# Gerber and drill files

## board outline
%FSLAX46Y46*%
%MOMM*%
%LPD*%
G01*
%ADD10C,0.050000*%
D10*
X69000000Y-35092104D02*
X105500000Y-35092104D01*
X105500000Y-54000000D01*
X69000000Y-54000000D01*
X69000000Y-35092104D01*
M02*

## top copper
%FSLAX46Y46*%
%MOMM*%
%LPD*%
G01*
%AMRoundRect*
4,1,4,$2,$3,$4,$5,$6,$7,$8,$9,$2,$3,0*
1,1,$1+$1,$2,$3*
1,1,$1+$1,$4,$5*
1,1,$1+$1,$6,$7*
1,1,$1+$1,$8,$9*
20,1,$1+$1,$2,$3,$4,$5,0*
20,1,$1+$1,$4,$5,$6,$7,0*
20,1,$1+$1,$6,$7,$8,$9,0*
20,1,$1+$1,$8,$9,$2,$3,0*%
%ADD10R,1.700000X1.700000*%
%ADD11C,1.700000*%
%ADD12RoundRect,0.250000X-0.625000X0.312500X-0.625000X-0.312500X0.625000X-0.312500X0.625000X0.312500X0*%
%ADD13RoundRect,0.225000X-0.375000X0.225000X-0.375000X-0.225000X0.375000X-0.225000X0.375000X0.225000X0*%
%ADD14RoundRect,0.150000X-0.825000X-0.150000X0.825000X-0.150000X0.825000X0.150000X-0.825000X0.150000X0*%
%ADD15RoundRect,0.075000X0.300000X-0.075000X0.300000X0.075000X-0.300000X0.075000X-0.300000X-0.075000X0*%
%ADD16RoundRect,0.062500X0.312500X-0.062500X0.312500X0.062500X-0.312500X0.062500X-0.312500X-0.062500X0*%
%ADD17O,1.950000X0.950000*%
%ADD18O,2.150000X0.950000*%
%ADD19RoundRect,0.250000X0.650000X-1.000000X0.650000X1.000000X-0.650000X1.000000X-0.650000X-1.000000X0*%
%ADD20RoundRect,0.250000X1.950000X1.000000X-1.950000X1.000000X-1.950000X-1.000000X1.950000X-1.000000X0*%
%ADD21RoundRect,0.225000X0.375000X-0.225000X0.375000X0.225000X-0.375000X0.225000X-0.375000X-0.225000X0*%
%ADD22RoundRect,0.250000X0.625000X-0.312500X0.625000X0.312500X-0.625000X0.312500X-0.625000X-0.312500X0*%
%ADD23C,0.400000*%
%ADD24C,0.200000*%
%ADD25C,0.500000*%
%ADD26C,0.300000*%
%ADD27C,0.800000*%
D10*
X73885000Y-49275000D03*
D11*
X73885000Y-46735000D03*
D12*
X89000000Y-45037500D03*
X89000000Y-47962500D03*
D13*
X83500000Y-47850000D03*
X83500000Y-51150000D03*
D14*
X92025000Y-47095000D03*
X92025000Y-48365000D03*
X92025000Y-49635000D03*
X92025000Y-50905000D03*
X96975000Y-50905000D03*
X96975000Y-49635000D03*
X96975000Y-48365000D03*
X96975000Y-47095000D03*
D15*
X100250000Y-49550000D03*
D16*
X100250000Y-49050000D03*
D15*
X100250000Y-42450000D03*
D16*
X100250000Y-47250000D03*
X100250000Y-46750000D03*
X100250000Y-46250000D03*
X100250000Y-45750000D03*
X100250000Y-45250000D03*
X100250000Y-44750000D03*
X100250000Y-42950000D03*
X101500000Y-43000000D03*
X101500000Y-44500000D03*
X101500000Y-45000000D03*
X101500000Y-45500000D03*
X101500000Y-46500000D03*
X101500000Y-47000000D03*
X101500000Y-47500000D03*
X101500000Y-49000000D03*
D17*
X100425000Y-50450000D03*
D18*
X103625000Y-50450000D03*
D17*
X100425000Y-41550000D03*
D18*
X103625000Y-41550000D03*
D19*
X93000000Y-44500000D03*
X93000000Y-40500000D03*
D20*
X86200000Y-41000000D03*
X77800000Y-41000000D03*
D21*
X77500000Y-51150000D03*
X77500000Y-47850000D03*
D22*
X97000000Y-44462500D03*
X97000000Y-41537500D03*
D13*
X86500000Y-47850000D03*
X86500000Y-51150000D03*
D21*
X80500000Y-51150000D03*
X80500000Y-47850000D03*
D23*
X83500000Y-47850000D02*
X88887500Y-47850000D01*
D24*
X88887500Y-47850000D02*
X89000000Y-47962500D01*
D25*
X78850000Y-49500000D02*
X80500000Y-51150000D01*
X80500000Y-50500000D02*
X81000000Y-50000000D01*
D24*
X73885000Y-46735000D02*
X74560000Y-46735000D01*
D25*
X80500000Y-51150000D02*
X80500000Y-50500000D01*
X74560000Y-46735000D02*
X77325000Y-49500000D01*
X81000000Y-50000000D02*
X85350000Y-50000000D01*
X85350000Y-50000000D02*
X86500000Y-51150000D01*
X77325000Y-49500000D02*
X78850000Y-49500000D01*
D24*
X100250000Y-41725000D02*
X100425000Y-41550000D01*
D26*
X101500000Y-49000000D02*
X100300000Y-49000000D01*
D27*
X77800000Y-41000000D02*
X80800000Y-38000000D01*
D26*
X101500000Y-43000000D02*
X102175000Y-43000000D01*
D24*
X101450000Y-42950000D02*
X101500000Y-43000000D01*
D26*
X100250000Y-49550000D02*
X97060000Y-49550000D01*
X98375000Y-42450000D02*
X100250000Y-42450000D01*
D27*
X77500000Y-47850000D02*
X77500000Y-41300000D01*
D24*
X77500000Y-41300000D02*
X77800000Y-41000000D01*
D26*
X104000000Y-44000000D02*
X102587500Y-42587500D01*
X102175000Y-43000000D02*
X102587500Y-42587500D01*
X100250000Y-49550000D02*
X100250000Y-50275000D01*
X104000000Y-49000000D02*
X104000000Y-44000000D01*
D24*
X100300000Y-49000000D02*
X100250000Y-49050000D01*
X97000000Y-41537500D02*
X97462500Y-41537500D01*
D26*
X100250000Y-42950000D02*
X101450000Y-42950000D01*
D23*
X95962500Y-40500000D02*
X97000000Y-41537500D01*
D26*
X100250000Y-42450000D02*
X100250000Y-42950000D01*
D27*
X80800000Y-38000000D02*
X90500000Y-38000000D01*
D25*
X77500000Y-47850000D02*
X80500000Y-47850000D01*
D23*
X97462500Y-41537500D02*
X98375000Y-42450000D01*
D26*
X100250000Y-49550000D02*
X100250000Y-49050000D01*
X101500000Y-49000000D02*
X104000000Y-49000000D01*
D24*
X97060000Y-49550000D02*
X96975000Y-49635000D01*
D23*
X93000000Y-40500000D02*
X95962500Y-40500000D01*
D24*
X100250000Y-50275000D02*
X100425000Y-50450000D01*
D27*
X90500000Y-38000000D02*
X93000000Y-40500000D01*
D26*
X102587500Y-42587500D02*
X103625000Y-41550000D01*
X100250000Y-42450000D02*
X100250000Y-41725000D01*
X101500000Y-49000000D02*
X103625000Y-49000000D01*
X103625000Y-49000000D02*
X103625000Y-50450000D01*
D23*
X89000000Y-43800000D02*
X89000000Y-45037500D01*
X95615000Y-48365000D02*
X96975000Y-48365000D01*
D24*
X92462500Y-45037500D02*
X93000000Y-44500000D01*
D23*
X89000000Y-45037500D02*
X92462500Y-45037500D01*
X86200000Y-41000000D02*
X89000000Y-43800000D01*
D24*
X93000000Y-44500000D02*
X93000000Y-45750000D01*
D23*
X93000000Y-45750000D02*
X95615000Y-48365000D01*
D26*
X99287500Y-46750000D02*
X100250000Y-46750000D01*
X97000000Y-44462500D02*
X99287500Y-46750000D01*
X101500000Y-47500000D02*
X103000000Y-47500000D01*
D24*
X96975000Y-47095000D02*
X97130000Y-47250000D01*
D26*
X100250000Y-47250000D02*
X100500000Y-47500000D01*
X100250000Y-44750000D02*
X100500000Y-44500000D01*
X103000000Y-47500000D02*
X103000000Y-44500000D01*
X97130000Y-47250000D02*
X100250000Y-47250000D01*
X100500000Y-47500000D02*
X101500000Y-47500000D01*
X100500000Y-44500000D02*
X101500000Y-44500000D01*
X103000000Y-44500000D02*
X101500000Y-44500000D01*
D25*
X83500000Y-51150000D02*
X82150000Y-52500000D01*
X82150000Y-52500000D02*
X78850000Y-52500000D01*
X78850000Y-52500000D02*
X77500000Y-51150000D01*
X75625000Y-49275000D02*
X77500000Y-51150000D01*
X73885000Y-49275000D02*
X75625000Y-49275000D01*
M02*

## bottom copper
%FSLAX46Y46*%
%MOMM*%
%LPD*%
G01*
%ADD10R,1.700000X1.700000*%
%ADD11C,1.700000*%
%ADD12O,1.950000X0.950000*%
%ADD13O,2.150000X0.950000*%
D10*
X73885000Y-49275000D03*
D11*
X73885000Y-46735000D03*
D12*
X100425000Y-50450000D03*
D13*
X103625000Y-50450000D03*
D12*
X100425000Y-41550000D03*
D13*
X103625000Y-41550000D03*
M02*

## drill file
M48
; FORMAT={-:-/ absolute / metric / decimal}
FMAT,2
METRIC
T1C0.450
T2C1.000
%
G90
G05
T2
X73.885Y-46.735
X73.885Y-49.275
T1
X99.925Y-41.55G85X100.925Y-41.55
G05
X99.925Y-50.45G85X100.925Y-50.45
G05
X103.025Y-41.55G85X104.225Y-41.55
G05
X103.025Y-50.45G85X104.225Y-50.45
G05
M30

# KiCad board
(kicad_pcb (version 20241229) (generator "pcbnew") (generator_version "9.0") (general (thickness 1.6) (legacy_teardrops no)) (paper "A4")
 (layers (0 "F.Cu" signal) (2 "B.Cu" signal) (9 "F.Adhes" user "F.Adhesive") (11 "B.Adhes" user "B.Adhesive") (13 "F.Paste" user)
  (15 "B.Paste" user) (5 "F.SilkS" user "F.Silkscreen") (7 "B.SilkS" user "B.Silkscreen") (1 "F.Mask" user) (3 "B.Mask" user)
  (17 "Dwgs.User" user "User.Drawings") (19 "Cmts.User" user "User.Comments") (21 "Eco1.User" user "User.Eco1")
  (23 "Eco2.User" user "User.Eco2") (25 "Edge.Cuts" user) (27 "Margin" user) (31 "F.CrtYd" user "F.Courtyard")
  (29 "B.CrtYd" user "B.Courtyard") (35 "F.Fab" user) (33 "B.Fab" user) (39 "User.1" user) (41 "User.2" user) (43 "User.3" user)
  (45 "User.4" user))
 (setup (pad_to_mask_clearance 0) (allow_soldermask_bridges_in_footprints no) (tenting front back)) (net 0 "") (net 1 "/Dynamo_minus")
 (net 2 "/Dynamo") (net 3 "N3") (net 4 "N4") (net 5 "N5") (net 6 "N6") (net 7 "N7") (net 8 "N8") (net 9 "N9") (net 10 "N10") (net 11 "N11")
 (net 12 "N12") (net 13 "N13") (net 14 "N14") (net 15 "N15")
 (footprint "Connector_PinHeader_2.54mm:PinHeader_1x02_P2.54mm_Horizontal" (layer "F.Cu") (at 73.885 49.275 180)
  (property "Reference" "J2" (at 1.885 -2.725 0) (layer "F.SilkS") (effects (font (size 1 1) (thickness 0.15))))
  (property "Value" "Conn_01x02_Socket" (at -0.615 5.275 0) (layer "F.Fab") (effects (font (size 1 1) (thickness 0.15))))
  (pad "1" thru_hole rect (at 0 0 180) (size 1.7 1.7) (drill 1) (layers "*.Cu" "*.Mask") (remove_unused_layers no) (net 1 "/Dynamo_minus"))
  (pad "2" thru_hole circle (at 0 2.54 180) (size 1.7 1.7) (drill 1) (layers "*.Cu" "*.Mask") (remove_unused_layers no) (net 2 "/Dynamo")))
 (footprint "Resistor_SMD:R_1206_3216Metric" (layer "F.Cu") (at 89 46.5 -90)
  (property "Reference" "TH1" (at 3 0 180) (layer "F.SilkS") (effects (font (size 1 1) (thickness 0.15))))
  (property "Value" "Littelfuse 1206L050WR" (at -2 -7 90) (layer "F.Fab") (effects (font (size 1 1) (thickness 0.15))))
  (pad "1" smd roundrect (at -1.4625 0 270) (size 1.125 1.75) (layers "F.Cu" "F.Mask" "F.Paste") (roundrect_rratio 0.222222) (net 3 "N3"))
  (pad "2" smd roundrect (at 1.4625 0 270) (size 1.125 1.75) (layers "F.Cu" "F.Mask" "F.Paste") (roundrect_rratio 0.222222) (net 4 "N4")))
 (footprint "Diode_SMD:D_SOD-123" (layer "F.Cu") (at 83.5 49.5 -90)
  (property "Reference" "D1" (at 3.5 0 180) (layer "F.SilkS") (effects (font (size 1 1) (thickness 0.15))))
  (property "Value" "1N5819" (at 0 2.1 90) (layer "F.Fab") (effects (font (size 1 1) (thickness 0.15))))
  (pad "1" smd roundrect (at -1.65 0 270) (size 0.9 1.2) (layers "F.Cu" "F.Mask" "F.Paste") (roundrect_rratio 0.25) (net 4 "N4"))
  (pad "2" smd roundrect (at 1.65 0 270) (size 0.9 1.2) (layers "F.Cu" "F.Mask" "F.Paste") (roundrect_rratio 0.25) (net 1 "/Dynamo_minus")))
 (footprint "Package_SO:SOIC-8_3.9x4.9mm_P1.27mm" (layer "F.Cu") (at 94.5 49)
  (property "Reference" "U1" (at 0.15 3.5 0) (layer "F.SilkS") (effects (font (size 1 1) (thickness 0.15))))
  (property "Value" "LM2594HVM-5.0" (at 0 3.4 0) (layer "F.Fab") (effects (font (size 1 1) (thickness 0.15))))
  (pad "1" smd roundrect (at -2.475 -1.905) (size 1.95 0.6) (layers "F.Cu" "F.Mask" "F.Paste") (roundrect_rratio 0.25) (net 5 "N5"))
  (pad "2" smd roundrect (at -2.475 -0.635) (size 1.95 0.6) (layers "F.Cu" "F.Mask" "F.Paste") (roundrect_rratio 0.25) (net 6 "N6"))
  (pad "3" smd roundrect (at -2.475 0.635) (size 1.95 0.6) (layers "F.Cu" "F.Mask" "F.Paste") (roundrect_rratio 0.25) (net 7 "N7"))
  (pad "4" smd roundrect (at -2.475 1.905) (size 1.95 0.6) (layers "F.Cu" "F.Mask" "F.Paste") (roundrect_rratio 0.25) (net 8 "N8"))
  (pad "5" smd roundrect (at 2.475 1.905) (size 1.95 0.6) (layers "F.Cu" "F.Mask" "F.Paste") (roundrect_rratio 0.25) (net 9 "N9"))
  (pad "6" smd roundrect (at 2.475 0.635) (size 1.95 0.6) (layers "F.Cu" "F.Mask" "F.Paste") (roundrect_rratio 0.25) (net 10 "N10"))
  (pad "7" smd roundrect (at 2.475 -0.635) (size 1.95 0.6) (layers "F.Cu" "F.Mask" "F.Paste") (roundrect_rratio 0.25) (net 3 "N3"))
  (pad "8" smd roundrect (at 2.475 -1.905) (size 1.95 0.6) (layers "F.Cu" "F.Mask" "F.Paste") (roundrect_rratio 0.25) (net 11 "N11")))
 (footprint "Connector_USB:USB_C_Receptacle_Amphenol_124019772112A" (layer "F.Cu") (at 103.45 46 90)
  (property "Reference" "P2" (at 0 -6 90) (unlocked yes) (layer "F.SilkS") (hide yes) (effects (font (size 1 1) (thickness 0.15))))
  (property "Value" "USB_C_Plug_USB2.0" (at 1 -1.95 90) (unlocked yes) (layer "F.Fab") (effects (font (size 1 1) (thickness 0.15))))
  (pad "A1" smd roundrect (at -3.55 -3.2 90) (size 0.3 0.75) (layers "F.Cu" "F.Mask" "F.Paste") (roundrect_rratio 0.25) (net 10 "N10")
   (thermal_bridge_angle 45))
  (pad "A1" smd roundrect (at -3.05 -3.2 90) (size 0.25 0.75) (layers "F.Cu" "F.Mask" "F.Paste") (roundrect_rratio 0.25) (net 10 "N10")
   (thermal_bridge_angle 45))
  (pad "A1" smd roundrect (at 3.55 -3.2 90) (size 0.3 0.75) (layers "F.Cu" "F.Mask" "F.Paste") (roundrect_rratio 0.25) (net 10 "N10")
   (thermal_bridge_angle 45))
  (pad "A4" smd roundrect (at -1.25 -3.2 90) (size 0.25 0.75) (layers "F.Cu" "F.Mask" "F.Paste") (roundrect_rratio 0.25) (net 11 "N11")
   (thermal_bridge_angle 45))
  (pad "A5" smd roundrect (at -0.75 -3.2 90) (size 0.25 0.75) (layers "F.Cu" "F.Mask" "F.Paste") (roundrect_rratio 0.25) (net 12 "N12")
   (thermal_bridge_angle 45))
  (pad "A6" smd roundrect (at -0.25 -3.2 90) (size 0.25 0.75) (layers "F.Cu" "F.Mask" "F.Paste") (roundrect_rratio 0.25) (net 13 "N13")
   (thermal_bridge_angle 45))
  (pad "A7" smd roundrect (at 0.25 -3.2 90) (size 0.25 0.75) (layers "F.Cu" "F.Mask" "F.Paste") (roundrect_rratio 0.25) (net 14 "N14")
   (thermal_bridge_angle 45))
  (pad "A8" smd roundrect (at 0.75 -3.2 90) (size 0.25 0.75) (layers "F.Cu" "F.Mask" "F.Paste") (roundrect_rratio 0.25)
   (thermal_bridge_angle 45))
  (pad "A9" smd roundrect (at 1.25 -3.2 90) (size 0.25 0.75) (layers "F.Cu" "F.Mask" "F.Paste") (roundrect_rratio 0.25) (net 11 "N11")
   (thermal_bridge_angle 45))
  (pad "A12" smd roundrect (at 3.05 -3.2 90) (size 0.25 0.75) (layers "F.Cu" "F.Mask" "F.Paste") (roundrect_rratio 0.25) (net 10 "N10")
   (thermal_bridge_angle 45))
  (pad "B1" smd roundrect (at 3 -1.95 90) (size 0.25 0.75) (layers "F.Cu" "F.Mask" "F.Paste") (roundrect_rratio 0.25) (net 10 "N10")
   (thermal_bridge_angle 45))
  (pad "B4" smd roundrect (at 1.5 -1.95 90) (size 0.25 0.75) (layers "F.Cu" "F.Mask" "F.Paste") (roundrect_rratio 0.25) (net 11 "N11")
   (thermal_bridge_angle 45))
  (pad "B5" smd roundrect (at 1 -1.95 90) (size 0.25 0.75) (layers "F.Cu" "F.Mask" "F.Paste") (roundrect_rratio 0.25) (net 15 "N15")
   (thermal_bridge_angle 45))
  (pad "B6" smd roundrect (at 0.5 -1.95 90) (size 0.25 0.75) (layers "F.Cu" "F.Mask" "F.Paste") (roundrect_rratio 0.25)
   (thermal_bridge_angle 45))
  (pad "B7" smd roundrect (at -0.5 -1.95 90) (size 0.25 0.75) (layers "F.Cu" "F.Mask" "F.Paste") (roundrect_rratio 0.25)
   (thermal_bridge_angle 45))
  (pad "B8" smd roundrect (at -1 -1.95 90) (size 0.25 0.75) (layers "F.Cu" "F.Mask" "F.Paste") (roundrect_rratio 0.25)
   (thermal_bridge_angle 45))
  (pad "B9" smd roundrect (at -1.5 -1.95 90) (size 0.25 0.75) (layers "F.Cu" "F.Mask" "F.Paste") (roundrect_rratio 0.25) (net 11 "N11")
   (thermal_bridge_angle 45))
  (pad "B12" smd roundrect (at -3 -1.95 90) (size 0.25 0.75) (layers "F.Cu" "F.Mask" "F.Paste") (roundrect_rratio 0.25) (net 10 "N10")
   (thermal_bridge_angle 45))
  (pad "S1" thru_hole oval (at -4.45 -3.025 90) (size 0.95 1.95) (drill oval 0.45 1.45) (layers "*.Cu" "*.Mask") (remove_unused_layers no)
   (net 10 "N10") (thermal_bridge_angle 45))
  (pad "S1" thru_hole oval (at -4.45 0.175 90) (size 0.95 2.15) (drill oval 0.45 1.65) (layers "*.Cu" "*.Mask") (remove_unused_layers no)
   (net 10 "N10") (thermal_bridge_angle 45))
  (pad "S1" thru_hole oval (at 4.45 -3.025 90) (size 0.95 1.95) (drill oval 0.45 1.45) (layers "*.Cu" "*.Mask") (remove_unused_layers no)
   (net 10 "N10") (thermal_bridge_angle 45))
  (pad "S1" thru_hole oval (at 4.45 0.175 90) (size 0.95 2.15) (drill oval 0.45 1.65) (layers "*.Cu" "*.Mask") (remove_unused_layers no)
   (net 10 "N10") (thermal_bridge_angle 45)))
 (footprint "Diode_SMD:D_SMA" (layer "F.Cu") (at 93 42.5 90)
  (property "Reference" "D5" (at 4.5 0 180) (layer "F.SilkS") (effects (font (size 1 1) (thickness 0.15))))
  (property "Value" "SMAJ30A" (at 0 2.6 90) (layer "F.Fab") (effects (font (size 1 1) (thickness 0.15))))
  (pad "1" smd roundrect (at -2 0 90) (size 2.5 1.8) (layers "F.Cu" "F.Mask" "F.Paste") (roundrect_rratio 0.1388888889) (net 3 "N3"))
  (pad "2" smd roundrect (at 2 0 90) (size 2.5 1.8) (layers "F.Cu" "F.Mask" "F.Paste") (roundrect_rratio 0.1388888889) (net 10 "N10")))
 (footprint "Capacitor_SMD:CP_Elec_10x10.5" (layer "F.Cu") (at 82 41 180)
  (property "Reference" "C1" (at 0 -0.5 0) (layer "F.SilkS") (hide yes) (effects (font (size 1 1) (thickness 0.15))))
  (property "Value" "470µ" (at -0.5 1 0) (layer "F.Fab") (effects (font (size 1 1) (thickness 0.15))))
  (pad "1" smd roundrect (at -4.2 0 180) (size 4.4 2.5) (layers "F.Cu" "F.Mask" "F.Paste") (roundrect_rratio 0.1) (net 3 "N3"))
  (pad "2" smd roundrect (at 4.2 0 180) (size 4.4 2.5) (layers "F.Cu" "F.Mask" "F.Paste") (roundrect_rratio 0.1) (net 10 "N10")))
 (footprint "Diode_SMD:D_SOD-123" (layer "F.Cu") (at 77.5 49.5 90)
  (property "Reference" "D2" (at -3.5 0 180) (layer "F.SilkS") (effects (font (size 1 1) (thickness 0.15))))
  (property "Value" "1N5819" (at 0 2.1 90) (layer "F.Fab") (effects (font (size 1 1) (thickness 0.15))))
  (pad "1" smd roundrect (at -1.65 0 90) (size 0.9 1.2) (layers "F.Cu" "F.Mask" "F.Paste") (roundrect_rratio 0.25) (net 1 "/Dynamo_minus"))
  (pad "2" smd roundrect (at 1.65 0 90) (size 0.9 1.2) (layers "F.Cu" "F.Mask" "F.Paste") (roundrect_rratio 0.25) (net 10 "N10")))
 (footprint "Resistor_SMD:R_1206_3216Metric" (layer "F.Cu") (at 97 43 90)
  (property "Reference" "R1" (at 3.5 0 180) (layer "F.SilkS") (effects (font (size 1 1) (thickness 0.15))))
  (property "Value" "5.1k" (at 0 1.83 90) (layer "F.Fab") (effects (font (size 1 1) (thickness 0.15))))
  (pad "1" smd roundrect (at -1.4625 0 90) (size 1.125 1.75) (layers "F.Cu" "F.Mask" "F.Paste") (roundrect_rratio 0.222222) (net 12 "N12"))
  (pad "2" smd roundrect (at 1.4625 0 90) (size 1.125 1.75) (layers "F.Cu" "F.Mask" "F.Paste") (roundrect_rratio 0.222222) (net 10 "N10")))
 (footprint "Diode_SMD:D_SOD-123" (layer "F.Cu") (at 86.5 49.5 -90)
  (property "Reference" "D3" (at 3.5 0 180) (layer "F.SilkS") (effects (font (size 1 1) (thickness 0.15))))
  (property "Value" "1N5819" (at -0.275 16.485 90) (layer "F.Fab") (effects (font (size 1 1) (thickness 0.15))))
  (pad "1" smd roundrect (at -1.65 0 270) (size 0.9 1.2) (layers "F.Cu" "F.Mask" "F.Paste") (roundrect_rratio 0.25) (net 4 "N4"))
  (pad "2" smd roundrect (at 1.65 0 270) (size 0.9 1.2) (layers "F.Cu" "F.Mask" "F.Paste") (roundrect_rratio 0.25) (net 2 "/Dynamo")))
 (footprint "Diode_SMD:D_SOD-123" (layer "F.Cu") (at 80.5 49.5 90)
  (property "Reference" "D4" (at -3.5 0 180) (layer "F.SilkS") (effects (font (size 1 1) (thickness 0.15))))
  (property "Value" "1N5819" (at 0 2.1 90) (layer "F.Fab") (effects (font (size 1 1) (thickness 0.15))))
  (pad "1" smd roundrect (at -1.65 0 90) (size 0.9 1.2) (layers "F.Cu" "F.Mask" "F.Paste") (roundrect_rratio 0.25) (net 2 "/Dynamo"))
  (pad "2" smd roundrect (at 1.65 0 90) (size 0.9 1.2) (layers "F.Cu" "F.Mask" "F.Paste") (roundrect_rratio 0.25) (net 10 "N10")))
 (gr_rect (start 69 35.092104) (end 105.5 54) (stroke (width 0.05) (type default)) (fill no) (layer "Edge.Cuts"))
 (segment (start 83.5 47.85) (end 88.8875 47.85) (width 0.4) (layer "F.Cu") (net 4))
 (segment (start 88.8875 47.85) (end 89 47.9625) (width 0.2) (layer "F.Cu") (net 4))
 (segment (start 78.85 49.5) (end 80.5 51.15) (width 0.5) (layer "F.Cu") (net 2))
 (segment (start 80.5 50.5) (end 81 50) (width 0.5) (layer "F.Cu") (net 2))
 (segment (start 73.885 46.735) (end 74.56 46.735) (width 0.2) (layer "F.Cu") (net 2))
 (segment (start 80.5 51.15) (end 80.5 50.5) (width 0.5) (layer "F.Cu") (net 2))
 (segment (start 74.56 46.735) (end 77.325 49.5) (width 0.5) (layer "F.Cu") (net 2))
 (segment (start 81 50) (end 85.35 50) (width 0.5) (layer "F.Cu") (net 2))
 (segment (start 85.35 50) (end 86.5 51.15) (width 0.5) (layer "F.Cu") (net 2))
 (segment (start 77.325 49.5) (end 78.85 49.5) (width 0.5) (layer "F.Cu") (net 2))
 (segment (start 100.25 41.725) (end 100.425 41.55) (width 0.2) (layer "F.Cu") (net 10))
 (segment (start 101.5 49) (end 100.3 49) (width 0.3) (layer "F.Cu") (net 10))
 (segment (start 77.8 41) (end 80.8 38) (width 0.8) (layer "F.Cu") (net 10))
 (segment (start 101.5 43) (end 102.175 43) (width 0.3) (layer "F.Cu") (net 10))
 (segment (start 101.45 42.95) (end 101.5 43) (width 0.2) (layer "F.Cu") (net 10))
 (segment (start 100.25 49.55) (end 97.06 49.55) (width 0.3) (layer "F.Cu") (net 10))
 (segment (start 98.375 42.45) (end 100.25 42.45) (width 0.3) (layer "F.Cu") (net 10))
 (segment (start 77.5 47.85) (end 77.5 41.3) (width 0.8) (layer "F.Cu") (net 10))
 (segment (start 77.5 41.3) (end 77.8 41) (width 0.2) (layer "F.Cu") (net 10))
 (segment (start 104 44) (end 102.5875 42.5875) (width 0.3) (layer "F.Cu") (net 10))
 (segment (start 102.175 43) (end 102.5875 42.5875) (width 0.3) (layer "F.Cu") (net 10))
 (segment (start 100.25 49.55) (end 100.25 50.275) (width 0.3) (layer "F.Cu") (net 10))
 (segment (start 104 49) (end 104 44) (width 0.3) (layer "F.Cu") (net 10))
 (segment (start 100.3 49) (end 100.25 49.05) (width 0.2) (layer "F.Cu") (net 10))
 (segment (start 97 41.5375) (end 97.4625 41.5375) (width 0.2) (layer "F.Cu") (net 10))
 (segment (start 100.25 42.95) (end 101.45 42.95) (width 0.3) (layer "F.Cu") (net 10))
 (segment (start 95.9625 40.5) (end 97 41.5375) (width 0.4) (layer "F.Cu") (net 10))
 (segment (start 100.25 42.45) (end 100.25 42.95) (width 0.3) (layer "F.Cu") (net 10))
 (segment (start 80.8 38) (end 90.5 38) (width 0.8) (layer "F.Cu") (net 10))
 (segment (start 77.5 47.85) (end 80.5 47.85) (width 0.5) (layer "F.Cu") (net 10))
 (segment (start 97.4625 41.5375) (end 98.375 42.45) (width 0.4) (layer "F.Cu") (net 10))
 (segment (start 100.25 49.55) (end 100.25 49.05) (width 0.3) (layer "F.Cu") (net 10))
 (segment (start 101.5 49) (end 104 49) (width 0.3) (layer "F.Cu") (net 10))
 (segment (start 97.06 49.55) (end 96.975 49.635) (width 0.2) (layer "F.Cu") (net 10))
 (segment (start 93 40.5) (end 95.9625 40.5) (width 0.4) (layer "F.Cu") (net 10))
 (segment (start 100.25 50.275) (end 100.425 50.45) (width 0.2) (layer "F.Cu") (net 10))
 (segment (start 90.5 38) (end 93 40.5) (width 0.8) (layer "F.Cu") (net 10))
 (segment (start 102.5875 42.5875) (end 103.625 41.55) (width 0.3) (layer "F.Cu") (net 10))
 (segment (start 100.25 42.45) (end 100.25 41.725) (width 0.3) (layer "F.Cu") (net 10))
 (segment (start 101.5 49) (end 103.625 49) (width 0.3) (layer "F.Cu") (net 10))
 (segment (start 103.625 49) (end 103.625 50.45) (width 0.3) (layer "F.Cu") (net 10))
 (segment (start 89 43.8) (end 89 45.0375) (width 0.4) (layer "F.Cu") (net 3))
 (segment (start 95.615 48.365) (end 96.975 48.365) (width 0.4) (layer "F.Cu") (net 3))
 (segment (start 92.4625 45.0375) (end 93 44.5) (width 0.2) (layer "F.Cu") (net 3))
 (segment (start 89 45.0375) (end 92.4625 45.0375) (width 0.4) (layer "F.Cu") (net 3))
 (segment (start 86.2 41) (end 89 43.8) (width 0.4) (layer "F.Cu") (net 3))
 (segment (start 93 44.5) (end 93 45.75) (width 0.2) (layer "F.Cu") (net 3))
 (segment (start 93 45.75) (end 95.615 48.365) (width 0.4) (layer "F.Cu") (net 3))
 (segment (start 99.2875 46.75) (end 100.25 46.75) (width 0.3) (layer "F.Cu") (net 12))
 (segment (start 97 44.4625) (end 99.2875 46.75) (width 0.3) (layer "F.Cu") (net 12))
 (segment (start 101.5 47.5) (end 103 47.5) (width 0.3) (layer "F.Cu") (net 11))
 (segment (start 96.975 47.095) (end 97.13 47.25) (width 0.2) (layer "F.Cu") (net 11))
 (segment (start 100.25 47.25) (end 100.5 47.5) (width 0.3) (layer "F.Cu") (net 11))
 (segment (start 100.25 44.75) (end 100.5 44.5) (width 0.3) (layer "F.Cu") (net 11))
 (segment (start 103 47.5) (end 103 44.5) (width 0.3) (layer "F.Cu") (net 11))
 (segment (start 97.13 47.25) (end 100.25 47.25) (width 0.3) (layer "F.Cu") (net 11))
 (segment (start 100.5 47.5) (end 101.5 47.5) (width 0.3) (layer "F.Cu") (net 11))
 (segment (start 100.5 44.5) (end 101.5 44.5) (width 0.3) (layer "F.Cu") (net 11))
 (segment (start 103 44.5) (end 101.5 44.5) (width 0.3) (layer "F.Cu") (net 11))
 (segment (start 83.5 51.15) (end 82.15 52.5) (width 0.5) (layer "F.Cu") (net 1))
 (segment (start 82.15 52.5) (end 78.85 52.5) (width 0.5) (layer "F.Cu") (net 1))
 (segment (start 78.85 52.5) (end 77.5 51.15) (width 0.5) (layer "F.Cu") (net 1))
 (segment (start 75.625 49.275) (end 77.5 51.15) (width 0.5) (layer "F.Cu") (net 1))
 (segment (start 73.885 49.275) (end 75.625 49.275) (width 0.5) (layer "F.Cu") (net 1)))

